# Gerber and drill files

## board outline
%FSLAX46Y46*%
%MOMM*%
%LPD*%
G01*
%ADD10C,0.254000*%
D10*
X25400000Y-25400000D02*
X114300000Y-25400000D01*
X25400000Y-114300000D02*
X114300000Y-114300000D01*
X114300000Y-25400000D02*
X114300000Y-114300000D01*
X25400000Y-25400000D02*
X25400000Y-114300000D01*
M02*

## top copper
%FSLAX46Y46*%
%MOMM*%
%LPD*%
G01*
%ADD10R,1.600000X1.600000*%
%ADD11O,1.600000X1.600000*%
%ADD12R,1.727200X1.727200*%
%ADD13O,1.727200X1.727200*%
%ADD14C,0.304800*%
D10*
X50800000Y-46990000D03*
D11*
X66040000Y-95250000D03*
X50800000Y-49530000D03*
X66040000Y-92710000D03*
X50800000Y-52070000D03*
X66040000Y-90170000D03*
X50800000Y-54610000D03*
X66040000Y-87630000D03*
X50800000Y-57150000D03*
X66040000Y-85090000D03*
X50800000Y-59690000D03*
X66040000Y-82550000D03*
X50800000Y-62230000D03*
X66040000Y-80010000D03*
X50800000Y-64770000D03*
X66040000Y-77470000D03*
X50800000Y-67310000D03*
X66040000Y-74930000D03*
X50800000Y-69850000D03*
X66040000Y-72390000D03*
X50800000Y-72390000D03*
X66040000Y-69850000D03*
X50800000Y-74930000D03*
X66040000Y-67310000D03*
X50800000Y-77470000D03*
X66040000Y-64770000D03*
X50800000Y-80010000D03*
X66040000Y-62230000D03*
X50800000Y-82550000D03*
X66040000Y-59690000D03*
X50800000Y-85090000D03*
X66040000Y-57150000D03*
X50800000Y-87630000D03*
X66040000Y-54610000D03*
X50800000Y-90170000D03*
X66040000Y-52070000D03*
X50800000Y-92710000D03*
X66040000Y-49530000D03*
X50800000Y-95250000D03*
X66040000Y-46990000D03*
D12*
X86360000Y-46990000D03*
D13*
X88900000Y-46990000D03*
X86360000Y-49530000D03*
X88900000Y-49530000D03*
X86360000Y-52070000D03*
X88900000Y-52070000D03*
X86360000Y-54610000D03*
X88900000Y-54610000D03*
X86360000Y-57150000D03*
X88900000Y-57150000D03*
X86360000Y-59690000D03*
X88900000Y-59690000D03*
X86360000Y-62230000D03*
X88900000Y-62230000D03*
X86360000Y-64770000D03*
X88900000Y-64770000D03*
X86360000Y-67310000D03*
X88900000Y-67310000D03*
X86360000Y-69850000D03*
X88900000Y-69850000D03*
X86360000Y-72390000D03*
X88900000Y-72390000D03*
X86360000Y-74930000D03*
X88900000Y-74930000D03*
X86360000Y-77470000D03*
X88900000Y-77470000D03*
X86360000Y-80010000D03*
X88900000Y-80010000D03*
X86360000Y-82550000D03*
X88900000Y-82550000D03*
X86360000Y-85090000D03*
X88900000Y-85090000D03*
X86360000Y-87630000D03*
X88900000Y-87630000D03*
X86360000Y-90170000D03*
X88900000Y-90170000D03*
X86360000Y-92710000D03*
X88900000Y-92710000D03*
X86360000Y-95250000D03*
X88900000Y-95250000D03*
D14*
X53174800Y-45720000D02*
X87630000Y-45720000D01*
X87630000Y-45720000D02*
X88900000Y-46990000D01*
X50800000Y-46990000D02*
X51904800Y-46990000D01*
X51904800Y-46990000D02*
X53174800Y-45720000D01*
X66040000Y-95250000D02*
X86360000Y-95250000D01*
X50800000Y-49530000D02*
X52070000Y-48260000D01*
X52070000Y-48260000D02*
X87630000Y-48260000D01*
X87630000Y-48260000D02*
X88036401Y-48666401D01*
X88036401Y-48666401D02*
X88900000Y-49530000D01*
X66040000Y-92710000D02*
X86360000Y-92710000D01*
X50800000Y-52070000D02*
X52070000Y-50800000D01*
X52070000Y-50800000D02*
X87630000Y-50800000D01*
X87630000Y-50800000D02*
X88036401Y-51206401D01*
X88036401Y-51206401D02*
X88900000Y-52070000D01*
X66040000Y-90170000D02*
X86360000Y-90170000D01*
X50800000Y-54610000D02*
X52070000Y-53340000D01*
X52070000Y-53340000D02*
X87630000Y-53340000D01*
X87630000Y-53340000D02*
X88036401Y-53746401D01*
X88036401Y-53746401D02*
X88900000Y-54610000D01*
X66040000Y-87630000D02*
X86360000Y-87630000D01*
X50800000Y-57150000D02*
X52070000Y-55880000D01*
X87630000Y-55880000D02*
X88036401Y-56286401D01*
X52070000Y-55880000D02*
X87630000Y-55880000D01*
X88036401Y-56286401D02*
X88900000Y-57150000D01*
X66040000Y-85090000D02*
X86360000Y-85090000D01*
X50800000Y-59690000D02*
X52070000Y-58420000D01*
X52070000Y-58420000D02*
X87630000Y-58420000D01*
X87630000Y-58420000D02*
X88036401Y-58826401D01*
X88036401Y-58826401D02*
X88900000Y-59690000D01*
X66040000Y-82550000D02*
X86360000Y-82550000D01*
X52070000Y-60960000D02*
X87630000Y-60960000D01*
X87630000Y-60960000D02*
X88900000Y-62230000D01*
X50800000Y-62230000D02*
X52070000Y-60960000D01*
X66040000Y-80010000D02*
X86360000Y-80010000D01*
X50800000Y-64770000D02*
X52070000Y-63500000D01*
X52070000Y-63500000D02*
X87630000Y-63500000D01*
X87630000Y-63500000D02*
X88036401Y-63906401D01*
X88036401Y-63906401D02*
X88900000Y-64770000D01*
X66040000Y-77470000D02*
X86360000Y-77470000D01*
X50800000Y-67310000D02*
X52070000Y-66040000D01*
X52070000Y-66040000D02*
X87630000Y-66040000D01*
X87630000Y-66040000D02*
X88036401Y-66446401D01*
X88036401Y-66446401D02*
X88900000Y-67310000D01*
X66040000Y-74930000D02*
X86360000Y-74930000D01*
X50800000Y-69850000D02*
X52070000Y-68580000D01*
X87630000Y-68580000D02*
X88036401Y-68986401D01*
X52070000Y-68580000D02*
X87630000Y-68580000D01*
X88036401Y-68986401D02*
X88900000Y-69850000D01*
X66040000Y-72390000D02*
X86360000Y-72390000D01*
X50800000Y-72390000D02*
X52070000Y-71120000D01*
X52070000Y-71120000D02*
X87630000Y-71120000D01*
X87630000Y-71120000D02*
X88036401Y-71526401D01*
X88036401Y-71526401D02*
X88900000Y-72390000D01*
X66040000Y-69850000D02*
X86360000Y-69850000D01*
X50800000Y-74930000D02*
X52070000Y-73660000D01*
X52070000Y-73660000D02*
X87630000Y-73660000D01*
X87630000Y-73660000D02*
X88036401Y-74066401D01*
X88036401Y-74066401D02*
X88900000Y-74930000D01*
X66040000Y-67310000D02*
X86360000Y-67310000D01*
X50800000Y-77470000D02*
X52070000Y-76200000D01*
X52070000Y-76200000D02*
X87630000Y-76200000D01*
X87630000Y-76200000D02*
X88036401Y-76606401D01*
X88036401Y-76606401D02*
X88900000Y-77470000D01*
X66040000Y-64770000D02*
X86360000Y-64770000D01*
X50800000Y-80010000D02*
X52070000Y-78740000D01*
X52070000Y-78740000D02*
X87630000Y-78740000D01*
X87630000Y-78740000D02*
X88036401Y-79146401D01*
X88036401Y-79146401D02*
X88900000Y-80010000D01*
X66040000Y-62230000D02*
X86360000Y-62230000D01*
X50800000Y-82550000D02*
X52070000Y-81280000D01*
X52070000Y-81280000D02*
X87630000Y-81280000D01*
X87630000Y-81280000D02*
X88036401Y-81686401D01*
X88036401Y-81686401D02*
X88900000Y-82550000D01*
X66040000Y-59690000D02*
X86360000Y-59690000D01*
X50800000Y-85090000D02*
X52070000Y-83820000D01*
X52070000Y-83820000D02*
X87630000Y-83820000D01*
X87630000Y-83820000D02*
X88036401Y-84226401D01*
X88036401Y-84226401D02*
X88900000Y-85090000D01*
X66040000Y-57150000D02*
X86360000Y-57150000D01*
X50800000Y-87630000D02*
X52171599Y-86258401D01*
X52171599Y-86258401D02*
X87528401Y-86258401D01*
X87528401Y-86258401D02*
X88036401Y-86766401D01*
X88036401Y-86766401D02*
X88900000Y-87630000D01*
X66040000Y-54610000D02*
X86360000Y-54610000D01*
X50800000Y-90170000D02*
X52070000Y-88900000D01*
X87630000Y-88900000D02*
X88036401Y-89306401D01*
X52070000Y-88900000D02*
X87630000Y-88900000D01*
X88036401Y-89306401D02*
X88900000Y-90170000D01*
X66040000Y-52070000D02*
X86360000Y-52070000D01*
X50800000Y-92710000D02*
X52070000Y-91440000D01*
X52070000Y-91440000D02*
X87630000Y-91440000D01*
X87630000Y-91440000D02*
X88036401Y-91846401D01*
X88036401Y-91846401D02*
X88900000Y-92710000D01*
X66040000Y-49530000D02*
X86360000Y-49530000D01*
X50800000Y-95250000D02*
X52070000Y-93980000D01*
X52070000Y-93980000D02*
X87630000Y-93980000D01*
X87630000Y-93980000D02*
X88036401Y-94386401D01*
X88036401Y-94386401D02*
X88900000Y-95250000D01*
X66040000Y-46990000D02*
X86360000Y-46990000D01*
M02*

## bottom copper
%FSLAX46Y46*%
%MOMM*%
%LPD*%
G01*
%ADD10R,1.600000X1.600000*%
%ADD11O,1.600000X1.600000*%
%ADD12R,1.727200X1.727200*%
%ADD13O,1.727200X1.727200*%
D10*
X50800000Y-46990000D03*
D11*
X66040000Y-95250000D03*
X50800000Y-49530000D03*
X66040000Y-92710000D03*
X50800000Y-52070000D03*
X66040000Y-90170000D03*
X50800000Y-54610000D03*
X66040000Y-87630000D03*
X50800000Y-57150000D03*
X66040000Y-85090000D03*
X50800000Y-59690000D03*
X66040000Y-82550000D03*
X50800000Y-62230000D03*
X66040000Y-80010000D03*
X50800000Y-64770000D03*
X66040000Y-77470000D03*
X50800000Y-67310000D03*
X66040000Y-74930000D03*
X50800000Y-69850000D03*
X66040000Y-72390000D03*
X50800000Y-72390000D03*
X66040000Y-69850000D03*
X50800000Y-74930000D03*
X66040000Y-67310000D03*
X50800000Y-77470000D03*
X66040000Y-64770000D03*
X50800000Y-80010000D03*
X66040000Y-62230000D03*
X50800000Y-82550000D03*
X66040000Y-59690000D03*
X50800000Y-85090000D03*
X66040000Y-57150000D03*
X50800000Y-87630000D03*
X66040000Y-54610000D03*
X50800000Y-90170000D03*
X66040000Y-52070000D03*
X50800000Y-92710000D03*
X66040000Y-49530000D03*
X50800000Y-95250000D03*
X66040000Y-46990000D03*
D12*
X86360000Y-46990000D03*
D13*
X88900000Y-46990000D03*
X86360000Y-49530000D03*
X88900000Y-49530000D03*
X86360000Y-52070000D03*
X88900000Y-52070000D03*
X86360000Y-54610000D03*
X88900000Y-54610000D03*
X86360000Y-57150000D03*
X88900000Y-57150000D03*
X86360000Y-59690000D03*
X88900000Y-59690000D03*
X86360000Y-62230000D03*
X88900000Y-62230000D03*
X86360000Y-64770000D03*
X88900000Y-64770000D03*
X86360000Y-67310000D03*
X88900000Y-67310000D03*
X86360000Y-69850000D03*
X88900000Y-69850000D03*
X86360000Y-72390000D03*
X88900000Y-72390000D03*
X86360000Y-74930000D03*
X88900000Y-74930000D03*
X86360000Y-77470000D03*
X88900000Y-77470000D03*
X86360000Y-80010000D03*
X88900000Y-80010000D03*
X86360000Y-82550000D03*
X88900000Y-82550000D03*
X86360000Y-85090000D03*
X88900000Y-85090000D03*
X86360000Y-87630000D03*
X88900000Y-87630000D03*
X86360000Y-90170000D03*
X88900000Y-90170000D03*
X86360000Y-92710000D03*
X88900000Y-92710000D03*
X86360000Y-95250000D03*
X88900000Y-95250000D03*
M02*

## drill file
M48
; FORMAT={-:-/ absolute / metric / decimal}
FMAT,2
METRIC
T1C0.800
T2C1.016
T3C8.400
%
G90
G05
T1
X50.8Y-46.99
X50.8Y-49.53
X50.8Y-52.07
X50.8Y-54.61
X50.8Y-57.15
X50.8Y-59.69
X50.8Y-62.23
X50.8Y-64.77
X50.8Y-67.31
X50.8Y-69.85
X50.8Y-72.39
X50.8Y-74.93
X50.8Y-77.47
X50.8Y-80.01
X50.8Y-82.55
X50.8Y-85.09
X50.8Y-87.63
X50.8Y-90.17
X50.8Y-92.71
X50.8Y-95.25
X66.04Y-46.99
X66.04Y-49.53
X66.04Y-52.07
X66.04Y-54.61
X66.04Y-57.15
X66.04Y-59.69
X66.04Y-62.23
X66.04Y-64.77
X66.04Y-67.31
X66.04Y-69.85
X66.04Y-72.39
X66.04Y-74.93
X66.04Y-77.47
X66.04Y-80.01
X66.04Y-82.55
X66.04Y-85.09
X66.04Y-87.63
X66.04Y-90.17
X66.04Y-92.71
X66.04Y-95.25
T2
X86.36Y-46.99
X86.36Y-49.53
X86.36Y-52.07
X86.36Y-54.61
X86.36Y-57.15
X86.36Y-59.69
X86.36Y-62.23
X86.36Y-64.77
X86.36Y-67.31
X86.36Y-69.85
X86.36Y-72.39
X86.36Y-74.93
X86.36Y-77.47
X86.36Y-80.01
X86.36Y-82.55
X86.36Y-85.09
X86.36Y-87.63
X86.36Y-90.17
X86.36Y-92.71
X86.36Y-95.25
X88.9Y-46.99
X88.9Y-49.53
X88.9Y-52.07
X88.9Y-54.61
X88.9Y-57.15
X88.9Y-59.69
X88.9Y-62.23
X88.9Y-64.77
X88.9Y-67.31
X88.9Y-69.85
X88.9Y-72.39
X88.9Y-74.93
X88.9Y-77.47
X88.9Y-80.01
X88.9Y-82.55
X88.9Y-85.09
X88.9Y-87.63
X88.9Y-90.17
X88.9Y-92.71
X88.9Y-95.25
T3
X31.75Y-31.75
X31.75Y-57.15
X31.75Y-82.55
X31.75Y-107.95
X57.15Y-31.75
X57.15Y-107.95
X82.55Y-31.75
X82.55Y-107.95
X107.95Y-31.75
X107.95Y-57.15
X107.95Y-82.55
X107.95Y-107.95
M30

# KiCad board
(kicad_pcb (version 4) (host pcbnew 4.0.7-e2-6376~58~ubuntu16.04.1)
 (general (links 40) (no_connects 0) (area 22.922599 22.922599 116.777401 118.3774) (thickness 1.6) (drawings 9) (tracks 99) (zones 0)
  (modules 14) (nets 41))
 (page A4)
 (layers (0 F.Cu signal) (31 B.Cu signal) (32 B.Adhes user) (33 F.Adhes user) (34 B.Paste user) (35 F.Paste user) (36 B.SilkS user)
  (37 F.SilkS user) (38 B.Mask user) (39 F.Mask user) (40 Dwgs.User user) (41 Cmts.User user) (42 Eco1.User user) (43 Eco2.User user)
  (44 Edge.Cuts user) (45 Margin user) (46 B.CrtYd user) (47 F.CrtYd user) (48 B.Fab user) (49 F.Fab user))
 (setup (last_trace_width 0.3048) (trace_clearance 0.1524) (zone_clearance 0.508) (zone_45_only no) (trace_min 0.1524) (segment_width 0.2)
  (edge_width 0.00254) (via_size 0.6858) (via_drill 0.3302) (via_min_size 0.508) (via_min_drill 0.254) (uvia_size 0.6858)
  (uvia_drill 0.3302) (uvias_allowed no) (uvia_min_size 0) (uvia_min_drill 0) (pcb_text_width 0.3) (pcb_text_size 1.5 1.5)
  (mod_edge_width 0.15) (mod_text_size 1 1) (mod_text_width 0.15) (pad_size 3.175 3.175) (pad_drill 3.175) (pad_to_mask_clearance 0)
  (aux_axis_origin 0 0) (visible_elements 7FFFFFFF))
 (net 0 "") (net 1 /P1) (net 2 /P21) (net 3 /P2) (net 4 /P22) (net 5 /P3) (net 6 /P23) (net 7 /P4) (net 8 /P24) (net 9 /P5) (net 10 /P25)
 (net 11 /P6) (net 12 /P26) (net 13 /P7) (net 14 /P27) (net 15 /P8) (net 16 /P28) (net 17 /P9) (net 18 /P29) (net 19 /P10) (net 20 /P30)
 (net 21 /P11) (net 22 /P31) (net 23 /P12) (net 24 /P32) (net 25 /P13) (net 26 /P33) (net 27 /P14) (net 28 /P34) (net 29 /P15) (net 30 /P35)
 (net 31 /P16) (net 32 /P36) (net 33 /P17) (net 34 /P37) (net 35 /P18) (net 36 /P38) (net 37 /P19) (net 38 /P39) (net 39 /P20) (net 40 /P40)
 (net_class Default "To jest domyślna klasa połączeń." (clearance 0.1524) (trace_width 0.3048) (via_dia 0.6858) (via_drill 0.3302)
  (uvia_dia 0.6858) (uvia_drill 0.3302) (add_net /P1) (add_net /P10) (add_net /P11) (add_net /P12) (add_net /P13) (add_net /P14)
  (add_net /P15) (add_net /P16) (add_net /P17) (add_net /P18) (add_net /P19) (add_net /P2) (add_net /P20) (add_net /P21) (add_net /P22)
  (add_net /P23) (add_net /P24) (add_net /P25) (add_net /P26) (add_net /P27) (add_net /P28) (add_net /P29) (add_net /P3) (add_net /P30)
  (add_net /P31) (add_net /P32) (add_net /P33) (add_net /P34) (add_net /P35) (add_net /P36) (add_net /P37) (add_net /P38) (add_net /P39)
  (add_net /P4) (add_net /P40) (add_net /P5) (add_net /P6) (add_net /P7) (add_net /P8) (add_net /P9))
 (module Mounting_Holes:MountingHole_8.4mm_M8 (layer F.Cu) (at 82.55 107.95)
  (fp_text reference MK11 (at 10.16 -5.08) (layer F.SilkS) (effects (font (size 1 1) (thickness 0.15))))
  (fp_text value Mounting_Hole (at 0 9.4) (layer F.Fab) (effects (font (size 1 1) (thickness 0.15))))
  (pad 1 np_thru_hole circle (at 0 0) (size 8.4 8.4) (drill 8.4) (layers *.Cu *.Mask)))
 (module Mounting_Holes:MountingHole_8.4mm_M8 (layer F.Cu) (at 57.15 107.95)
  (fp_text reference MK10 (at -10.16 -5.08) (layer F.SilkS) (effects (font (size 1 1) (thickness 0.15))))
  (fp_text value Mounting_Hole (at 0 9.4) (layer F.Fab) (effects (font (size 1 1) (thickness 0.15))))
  (pad 1 np_thru_hole circle (at 0 0) (size 8.4 8.4) (drill 8.4) (layers *.Cu *.Mask)))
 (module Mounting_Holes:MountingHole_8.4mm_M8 (layer F.Cu) (at 107.95 82.55)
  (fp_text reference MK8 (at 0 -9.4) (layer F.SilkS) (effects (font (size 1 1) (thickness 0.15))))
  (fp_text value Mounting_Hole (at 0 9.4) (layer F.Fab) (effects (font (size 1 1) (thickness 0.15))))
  (pad 1 np_thru_hole circle (at 0 0) (size 8.4 8.4) (drill 8.4) (layers *.Cu *.Mask)))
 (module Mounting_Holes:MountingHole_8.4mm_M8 (layer F.Cu) (at 107.95 57.15)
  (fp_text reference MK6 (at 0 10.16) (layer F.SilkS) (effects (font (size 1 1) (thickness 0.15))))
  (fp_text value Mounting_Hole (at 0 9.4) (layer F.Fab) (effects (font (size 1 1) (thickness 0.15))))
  (pad 1 np_thru_hole circle (at 0 0) (size 8.4 8.4) (drill 8.4) (layers *.Cu *.Mask)))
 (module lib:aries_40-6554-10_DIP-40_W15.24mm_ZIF (layer F.Cu) (at 50.8 46.99)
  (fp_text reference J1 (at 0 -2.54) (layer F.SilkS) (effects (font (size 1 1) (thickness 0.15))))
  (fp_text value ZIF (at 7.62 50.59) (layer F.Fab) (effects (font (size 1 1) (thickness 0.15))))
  (pad 1 thru_hole rect (at 0 0) (size 1.6 1.6) (drill 0.8) (layers *.Cu *.Mask) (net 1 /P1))
  (pad 21 thru_hole oval (at 15.24 48.26) (size 1.6 1.6) (drill 0.8) (layers *.Cu *.Mask) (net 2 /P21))
  (pad 2 thru_hole oval (at 0 2.54) (size 1.6 1.6) (drill 0.8) (layers *.Cu *.Mask) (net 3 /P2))
  (pad 22 thru_hole oval (at 15.24 45.72) (size 1.6 1.6) (drill 0.8) (layers *.Cu *.Mask) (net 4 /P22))
  (pad 3 thru_hole oval (at 0 5.08) (size 1.6 1.6) (drill 0.8) (layers *.Cu *.Mask) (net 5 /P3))
  (pad 23 thru_hole oval (at 15.24 43.18) (size 1.6 1.6) (drill 0.8) (layers *.Cu *.Mask) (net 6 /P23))
  (pad 4 thru_hole oval (at 0 7.62) (size 1.6 1.6) (drill 0.8) (layers *.Cu *.Mask) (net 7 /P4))
  (pad 24 thru_hole oval (at 15.24 40.64) (size 1.6 1.6) (drill 0.8) (layers *.Cu *.Mask) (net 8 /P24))
  (pad 5 thru_hole oval (at 0 10.16) (size 1.6 1.6) (drill 0.8) (layers *.Cu *.Mask) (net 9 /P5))
  (pad 25 thru_hole oval (at 15.24 38.1) (size 1.6 1.6) (drill 0.8) (layers *.Cu *.Mask) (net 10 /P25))
  (pad 6 thru_hole oval (at 0 12.7) (size 1.6 1.6) (drill 0.8) (layers *.Cu *.Mask) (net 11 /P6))
  (pad 26 thru_hole oval (at 15.24 35.56) (size 1.6 1.6) (drill 0.8) (layers *.Cu *.Mask) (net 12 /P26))
  (pad 7 thru_hole oval (at 0 15.24) (size 1.6 1.6) (drill 0.8) (layers *.Cu *.Mask) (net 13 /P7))
  (pad 27 thru_hole oval (at 15.24 33.02) (size 1.6 1.6) (drill 0.8) (layers *.Cu *.Mask) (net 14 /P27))
  (pad 8 thru_hole oval (at 0 17.78) (size 1.6 1.6) (drill 0.8) (layers *.Cu *.Mask) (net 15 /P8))
  (pad 28 thru_hole oval (at 15.24 30.48) (size 1.6 1.6) (drill 0.8) (layers *.Cu *.Mask) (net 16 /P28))
  (pad 9 thru_hole oval (at 0 20.32) (size 1.6 1.6) (drill 0.8) (layers *.Cu *.Mask) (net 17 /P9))
  (pad 29 thru_hole oval (at 15.24 27.94) (size 1.6 1.6) (drill 0.8) (layers *.Cu *.Mask) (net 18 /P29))
  (pad 10 thru_hole oval (at 0 22.86) (size 1.6 1.6) (drill 0.8) (layers *.Cu *.Mask) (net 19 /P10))
  (pad 30 thru_hole oval (at 15.24 25.4) (size 1.6 1.6) (drill 0.8) (layers *.Cu *.Mask) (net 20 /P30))
  (pad 11 thru_hole oval (at 0 25.4) (size 1.6 1.6) (drill 0.8) (layers *.Cu *.Mask) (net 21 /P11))
  (pad 31 thru_hole oval (at 15.24 22.86) (size 1.6 1.6) (drill 0.8) (layers *.Cu *.Mask) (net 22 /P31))
  (pad 12 thru_hole oval (at 0 27.94) (size 1.6 1.6) (drill 0.8) (layers *.Cu *.Mask) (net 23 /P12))
  (pad 32 thru_hole oval (at 15.24 20.32) (size 1.6 1.6) (drill 0.8) (layers *.Cu *.Mask) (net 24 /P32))
  (pad 13 thru_hole oval (at 0 30.48) (size 1.6 1.6) (drill 0.8) (layers *.Cu *.Mask) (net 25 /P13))
  (pad 33 thru_hole oval (at 15.24 17.78) (size 1.6 1.6) (drill 0.8) (layers *.Cu *.Mask) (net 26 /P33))
  (pad 14 thru_hole oval (at 0 33.02) (size 1.6 1.6) (drill 0.8) (layers *.Cu *.Mask) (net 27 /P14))
  (pad 34 thru_hole oval (at 15.24 15.24) (size 1.6 1.6) (drill 0.8) (layers *.Cu *.Mask) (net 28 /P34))
  (pad 15 thru_hole oval (at 0 35.56) (size 1.6 1.6) (drill 0.8) (layers *.Cu *.Mask) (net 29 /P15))
  (pad 35 thru_hole oval (at 15.24 12.7) (size 1.6 1.6) (drill 0.8) (layers *.Cu *.Mask) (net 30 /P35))
  (pad 16 thru_hole oval (at 0 38.1) (size 1.6 1.6) (drill 0.8) (layers *.Cu *.Mask) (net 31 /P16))
  (pad 36 thru_hole oval (at 15.24 10.16) (size 1.6 1.6) (drill 0.8) (layers *.Cu *.Mask) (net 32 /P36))
  (pad 17 thru_hole oval (at 0 40.64) (size 1.6 1.6) (drill 0.8) (layers *.Cu *.Mask) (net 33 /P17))
  (pad 37 thru_hole oval (at 15.24 7.62) (size 1.6 1.6) (drill 0.8) (layers *.Cu *.Mask) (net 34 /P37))
  (pad 18 thru_hole oval (at 0 43.18) (size 1.6 1.6) (drill 0.8) (layers *.Cu *.Mask) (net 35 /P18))
  (pad 38 thru_hole oval (at 15.24 5.08) (size 1.6 1.6) (drill 0.8) (layers *.Cu *.Mask) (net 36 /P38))
  (pad 19 thru_hole oval (at 0 45.72) (size 1.6 1.6) (drill 0.8) (layers *.Cu *.Mask) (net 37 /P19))
  (pad 39 thru_hole oval (at 15.24 2.54) (size 1.6 1.6) (drill 0.8) (layers *.Cu *.Mask) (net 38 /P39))
  (pad 20 thru_hole oval (at 0 48.26) (size 1.6 1.6) (drill 0.8) (layers *.Cu *.Mask) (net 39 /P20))
  (pad 40 thru_hole oval (at 15.24 0) (size 1.6 1.6) (drill 0.8) (layers *.Cu *.Mask) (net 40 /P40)))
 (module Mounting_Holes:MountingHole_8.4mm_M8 (layer F.Cu) (at 31.75 31.75)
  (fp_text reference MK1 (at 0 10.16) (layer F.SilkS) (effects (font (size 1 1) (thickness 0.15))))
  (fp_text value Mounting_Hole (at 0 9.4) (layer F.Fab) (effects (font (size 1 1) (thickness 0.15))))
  (pad 1 np_thru_hole circle (at 0 0) (size 8.4 8.4) (drill 8.4) (layers *.Cu *.Mask)))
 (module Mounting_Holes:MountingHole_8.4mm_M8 (layer F.Cu) (at 107.95 31.75)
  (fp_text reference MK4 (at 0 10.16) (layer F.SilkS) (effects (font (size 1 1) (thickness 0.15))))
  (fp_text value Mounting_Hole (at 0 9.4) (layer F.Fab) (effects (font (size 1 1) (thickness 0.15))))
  (pad 1 np_thru_hole circle (at 0 0) (size 8.4 8.4) (drill 8.4) (layers *.Cu *.Mask)))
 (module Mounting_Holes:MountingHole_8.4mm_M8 (layer F.Cu) (at 31.75 107.95)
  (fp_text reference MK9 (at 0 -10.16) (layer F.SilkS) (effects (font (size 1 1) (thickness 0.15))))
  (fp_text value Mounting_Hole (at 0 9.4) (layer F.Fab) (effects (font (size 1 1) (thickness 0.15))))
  (pad 1 np_thru_hole circle (at 0 0) (size 8.4 8.4) (drill 8.4) (layers *.Cu *.Mask)))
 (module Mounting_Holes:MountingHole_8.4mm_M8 (layer F.Cu) (at 107.95 107.95)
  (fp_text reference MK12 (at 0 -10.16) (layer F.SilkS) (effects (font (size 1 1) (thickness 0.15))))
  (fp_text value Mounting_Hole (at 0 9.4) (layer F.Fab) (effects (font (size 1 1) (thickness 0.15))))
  (pad 1 np_thru_hole circle (at 0 0) (size 8.4 8.4) (drill 8.4) (layers *.Cu *.Mask)))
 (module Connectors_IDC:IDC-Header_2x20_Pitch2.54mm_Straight (layer F.Cu) (at 86.36 46.99)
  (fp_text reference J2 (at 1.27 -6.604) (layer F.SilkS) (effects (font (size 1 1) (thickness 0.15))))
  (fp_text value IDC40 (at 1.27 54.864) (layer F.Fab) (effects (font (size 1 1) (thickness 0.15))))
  (pad 1 thru_hole rect (at 0 0) (size 1.7272 1.7272) (drill 1.016) (layers *.Cu *.Mask) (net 40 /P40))
  (pad 2 thru_hole oval (at 2.54 0) (size 1.7272 1.7272) (drill 1.016) (layers *.Cu *.Mask) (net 1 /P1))
  (pad 3 thru_hole oval (at 0 2.54) (size 1.7272 1.7272) (drill 1.016) (layers *.Cu *.Mask) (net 38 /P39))
  (pad 4 thru_hole oval (at 2.54 2.54) (size 1.7272 1.7272) (drill 1.016) (layers *.Cu *.Mask) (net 3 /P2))
  (pad 5 thru_hole oval (at 0 5.08) (size 1.7272 1.7272) (drill 1.016) (layers *.Cu *.Mask) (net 36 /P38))
  (pad 6 thru_hole oval (at 2.54 5.08) (size 1.7272 1.7272) (drill 1.016) (layers *.Cu *.Mask) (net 5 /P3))
  (pad 7 thru_hole oval (at 0 7.62) (size 1.7272 1.7272) (drill 1.016) (layers *.Cu *.Mask) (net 34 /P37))
  (pad 8 thru_hole oval (at 2.54 7.62) (size 1.7272 1.7272) (drill 1.016) (layers *.Cu *.Mask) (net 7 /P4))
  (pad 9 thru_hole oval (at 0 10.16) (size 1.7272 1.7272) (drill 1.016) (layers *.Cu *.Mask) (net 32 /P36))
  (pad 10 thru_hole oval (at 2.54 10.16) (size 1.7272 1.7272) (drill 1.016) (layers *.Cu *.Mask) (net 9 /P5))
  (pad 11 thru_hole oval (at 0 12.7) (size 1.7272 1.7272) (drill 1.016) (layers *.Cu *.Mask) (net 30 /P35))
  (pad 12 thru_hole oval (at 2.54 12.7) (size 1.7272 1.7272) (drill 1.016) (layers *.Cu *.Mask) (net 11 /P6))
  (pad 13 thru_hole oval (at 0 15.24) (size 1.7272 1.7272) (drill 1.016) (layers *.Cu *.Mask) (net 28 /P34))
  (pad 14 thru_hole oval (at 2.54 15.24) (size 1.7272 1.7272) (drill 1.016) (layers *.Cu *.Mask) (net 13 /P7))
  (pad 15 thru_hole oval (at 0 17.78) (size 1.7272 1.7272) (drill 1.016) (layers *.Cu *.Mask) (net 26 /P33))
  (pad 16 thru_hole oval (at 2.54 17.78) (size 1.7272 1.7272) (drill 1.016) (layers *.Cu *.Mask) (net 15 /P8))
  (pad 17 thru_hole oval (at 0 20.32) (size 1.7272 1.7272) (drill 1.016) (layers *.Cu *.Mask) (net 24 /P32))
  (pad 18 thru_hole oval (at 2.54 20.32) (size 1.7272 1.7272) (drill 1.016) (layers *.Cu *.Mask) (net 17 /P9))
  (pad 19 thru_hole oval (at 0 22.86) (size 1.7272 1.7272) (drill 1.016) (layers *.Cu *.Mask) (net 22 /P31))
  (pad 20 thru_hole oval (at 2.54 22.86) (size 1.7272 1.7272) (drill 1.016) (layers *.Cu *.Mask) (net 19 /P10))
  (pad 21 thru_hole oval (at 0 25.4) (size 1.7272 1.7272) (drill 1.016) (layers *.Cu *.Mask) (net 20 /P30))
  (pad 22 thru_hole oval (at 2.54 25.4) (size 1.7272 1.7272) (drill 1.016) (layers *.Cu *.Mask) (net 21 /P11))
  (pad 23 thru_hole oval (at 0 27.94) (size 1.7272 1.7272) (drill 1.016) (layers *.Cu *.Mask) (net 18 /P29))
  (pad 24 thru_hole oval (at 2.54 27.94) (size 1.7272 1.7272) (drill 1.016) (layers *.Cu *.Mask) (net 23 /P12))
  (pad 25 thru_hole oval (at 0 30.48) (size 1.7272 1.7272) (drill 1.016) (layers *.Cu *.Mask) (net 16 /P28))
  (pad 26 thru_hole oval (at 2.54 30.48) (size 1.7272 1.7272) (drill 1.016) (layers *.Cu *.Mask) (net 25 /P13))
  (pad 27 thru_hole oval (at 0 33.02) (size 1.7272 1.7272) (drill 1.016) (layers *.Cu *.Mask) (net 14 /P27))
  (pad 28 thru_hole oval (at 2.54 33.02) (size 1.7272 1.7272) (drill 1.016) (layers *.Cu *.Mask) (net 27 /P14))
  (pad 29 thru_hole oval (at 0 35.56) (size 1.7272 1.7272) (drill 1.016) (layers *.Cu *.Mask) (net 12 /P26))
  (pad 30 thru_hole oval (at 2.54 35.56) (size 1.7272 1.7272) (drill 1.016) (layers *.Cu *.Mask) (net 29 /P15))
  (pad 31 thru_hole oval (at 0 38.1) (size 1.7272 1.7272) (drill 1.016) (layers *.Cu *.Mask) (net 10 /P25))
  (pad 32 thru_hole oval (at 2.54 38.1) (size 1.7272 1.7272) (drill 1.016) (layers *.Cu *.Mask) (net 31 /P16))
  (pad 33 thru_hole oval (at 0 40.64) (size 1.7272 1.7272) (drill 1.016) (layers *.Cu *.Mask) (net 8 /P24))
  (pad 34 thru_hole oval (at 2.54 40.64) (size 1.7272 1.7272) (drill 1.016) (layers *.Cu *.Mask) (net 33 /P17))
  (pad 35 thru_hole oval (at 0 43.18) (size 1.7272 1.7272) (drill 1.016) (layers *.Cu *.Mask) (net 6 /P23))
  (pad 36 thru_hole oval (at 2.54 43.18) (size 1.7272 1.7272) (drill 1.016) (layers *.Cu *.Mask) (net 35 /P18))
  (pad 37 thru_hole oval (at 0 45.72) (size 1.7272 1.7272) (drill 1.016) (layers *.Cu *.Mask) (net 4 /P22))
  (pad 38 thru_hole oval (at 2.54 45.72) (size 1.7272 1.7272) (drill 1.016) (layers *.Cu *.Mask) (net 37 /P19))
  (pad 39 thru_hole oval (at 0 48.26) (size 1.7272 1.7272) (drill 1.016) (layers *.Cu *.Mask) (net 2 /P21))
  (pad 40 thru_hole oval (at 2.54 48.26) (size 1.7272 1.7272) (drill 1.016) (layers *.Cu *.Mask) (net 39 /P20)))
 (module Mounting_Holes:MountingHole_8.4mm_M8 (layer F.Cu) (at 82.55 31.75)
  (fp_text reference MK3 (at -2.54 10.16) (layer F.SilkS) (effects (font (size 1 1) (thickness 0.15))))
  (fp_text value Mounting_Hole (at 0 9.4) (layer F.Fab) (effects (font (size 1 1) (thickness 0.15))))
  (pad 1 np_thru_hole circle (at 0 0) (size 8.4 8.4) (drill 8.4) (layers *.Cu *.Mask)))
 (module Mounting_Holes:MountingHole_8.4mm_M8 (layer F.Cu) (at 57.15 31.75)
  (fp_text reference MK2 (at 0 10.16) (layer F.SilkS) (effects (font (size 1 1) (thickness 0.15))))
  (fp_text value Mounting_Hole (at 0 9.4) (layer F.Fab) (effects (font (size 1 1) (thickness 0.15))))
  (pad 1 np_thru_hole circle (at 0 0) (size 8.4 8.4) (drill 8.4) (layers *.Cu *.Mask)))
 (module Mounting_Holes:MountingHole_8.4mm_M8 (layer F.Cu) (at 31.75 57.15)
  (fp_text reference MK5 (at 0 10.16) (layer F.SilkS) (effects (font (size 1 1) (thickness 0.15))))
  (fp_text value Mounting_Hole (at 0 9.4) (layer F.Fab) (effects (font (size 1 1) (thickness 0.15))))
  (pad 1 np_thru_hole circle (at 0 0) (size 8.4 8.4) (drill 8.4) (layers *.Cu *.Mask)))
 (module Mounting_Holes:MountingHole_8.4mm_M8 (layer F.Cu) (at 31.75 82.55)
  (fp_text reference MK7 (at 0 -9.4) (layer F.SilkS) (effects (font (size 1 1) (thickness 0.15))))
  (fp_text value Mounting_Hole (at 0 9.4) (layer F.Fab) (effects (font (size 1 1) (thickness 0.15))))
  (pad 1 np_thru_hole circle (at 0 0) (size 8.4 8.4) (drill 8.4) (layers *.Cu *.Mask)))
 (gr_line (start 25.4 25.4) (end 114.3 25.4) (layer Edge.Cuts) (width 0.254))
 (gr_line (start 25.4 114.3) (end 114.3 114.3) (layer Edge.Cuts) (width 0.254))
 (gr_line (start 114.3 25.4) (end 114.3 114.3) (layer Edge.Cuts) (width 0.254))
 (gr_line (start 25.4 25.4) (end 25.4 114.3) (layer Edge.Cuts) (width 0.254))
 (segment (start 53.1748 45.72) (end 87.63 45.72) (width 0.3048) (layer F.Cu) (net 1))
 (segment (start 87.63 45.72) (end 88.9 46.99) (width 0.3048) (layer F.Cu) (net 1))
 (segment (start 50.8 46.99) (end 51.9048 46.99) (width 0.3048) (layer F.Cu) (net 1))
 (segment (start 51.9048 46.99) (end 53.1748 45.72) (width 0.3048) (layer F.Cu) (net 1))
 (segment (start 66.04 95.25) (end 86.36 95.25) (width 0.3048) (layer F.Cu) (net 2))
 (segment (start 50.8 49.53) (end 52.07 48.26) (width 0.3048) (layer F.Cu) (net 3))
 (segment (start 52.07 48.26) (end 87.63 48.26) (width 0.3048) (layer F.Cu) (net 3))
 (segment (start 87.63 48.26) (end 88.036401 48.666401) (width 0.3048) (layer F.Cu) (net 3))
 (segment (start 88.036401 48.666401) (end 88.9 49.53) (width 0.3048) (layer F.Cu) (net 3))
 (segment (start 66.04 92.71) (end 86.36 92.71) (width 0.3048) (layer F.Cu) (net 4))
 (segment (start 50.8 52.07) (end 52.07 50.8) (width 0.3048) (layer F.Cu) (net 5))
 (segment (start 52.07 50.8) (end 87.63 50.8) (width 0.3048) (layer F.Cu) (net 5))
 (segment (start 87.63 50.8) (end 88.036401 51.206401) (width 0.3048) (layer F.Cu) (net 5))
 (segment (start 88.036401 51.206401) (end 88.9 52.07) (width 0.3048) (layer F.Cu) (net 5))
 (segment (start 66.04 90.17) (end 86.36 90.17) (width 0.3048) (layer F.Cu) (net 6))
 (segment (start 50.8 54.61) (end 52.07 53.34) (width 0.3048) (layer F.Cu) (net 7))
 (segment (start 52.07 53.34) (end 87.63 53.34) (width 0.3048) (layer F.Cu) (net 7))
 (segment (start 87.63 53.34) (end 88.036401 53.746401) (width 0.3048) (layer F.Cu) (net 7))
 (segment (start 88.036401 53.746401) (end 88.9 54.61) (width 0.3048) (layer F.Cu) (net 7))
 (segment (start 66.04 87.63) (end 86.36 87.63) (width 0.3048) (layer F.Cu) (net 8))
 (segment (start 50.8 57.15) (end 52.07 55.88) (width 0.3048) (layer F.Cu) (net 9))
 (segment (start 87.63 55.88) (end 88.036401 56.286401) (width 0.3048) (layer F.Cu) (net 9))
 (segment (start 52.07 55.88) (end 87.63 55.88) (width 0.3048) (layer F.Cu) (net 9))
 (segment (start 88.036401 56.286401) (end 88.9 57.15) (width 0.3048) (layer F.Cu) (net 9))
 (segment (start 66.04 85.09) (end 86.36 85.09) (width 0.3048) (layer F.Cu) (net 10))
 (segment (start 50.8 59.69) (end 52.07 58.42) (width 0.3048) (layer F.Cu) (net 11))
 (segment (start 52.07 58.42) (end 87.63 58.42) (width 0.3048) (layer F.Cu) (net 11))
 (segment (start 87.63 58.42) (end 88.036401 58.826401) (width 0.3048) (layer F.Cu) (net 11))
 (segment (start 88.036401 58.826401) (end 88.9 59.69) (width 0.3048) (layer F.Cu) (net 11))
 (segment (start 66.04 82.55) (end 86.36 82.55) (width 0.3048) (layer F.Cu) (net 12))
 (segment (start 52.07 60.96) (end 87.63 60.96) (width 0.3048) (layer F.Cu) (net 13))
 (segment (start 87.63 60.96) (end 88.9 62.23) (width 0.3048) (layer F.Cu) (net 13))
 (segment (start 50.8 62.23) (end 52.07 60.96) (width 0.3048) (layer F.Cu) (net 13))
 (segment (start 66.04 80.01) (end 86.36 80.01) (width 0.3048) (layer F.Cu) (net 14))
 (segment (start 50.8 64.77) (end 52.07 63.5) (width 0.3048) (layer F.Cu) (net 15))
 (segment (start 52.07 63.5) (end 87.63 63.5) (width 0.3048) (layer F.Cu) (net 15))
 (segment (start 87.63 63.5) (end 88.036401 63.906401) (width 0.3048) (layer F.Cu) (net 15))
 (segment (start 88.036401 63.906401) (end 88.9 64.77) (width 0.3048) (layer F.Cu) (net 15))
 (segment (start 66.04 77.47) (end 86.36 77.47) (width 0.3048) (layer F.Cu) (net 16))
 (segment (start 50.8 67.31) (end 52.07 66.04) (width 0.3048) (layer F.Cu) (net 17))
 (segment (start 52.07 66.04) (end 87.63 66.04) (width 0.3048) (layer F.Cu) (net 17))
 (segment (start 87.63 66.04) (end 88.036401 66.446401) (width 0.3048) (layer F.Cu) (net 17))
 (segment (start 88.036401 66.446401) (end 88.9 67.31) (width 0.3048) (layer F.Cu) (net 17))
 (segment (start 66.04 74.93) (end 86.36 74.93) (width 0.3048) (layer F.Cu) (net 18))
 (segment (start 50.8 69.85) (end 52.07 68.58) (width 0.3048) (layer F.Cu) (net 19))
 (segment (start 87.63 68.58) (end 88.036401 68.986401) (width 0.3048) (layer F.Cu) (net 19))
 (segment (start 52.07 68.58) (end 87.63 68.58) (width 0.3048) (layer F.Cu) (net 19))
 (segment (start 88.036401 68.986401) (end 88.9 69.85) (width 0.3048) (layer F.Cu) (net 19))
 (segment (start 66.04 72.39) (end 86.36 72.39) (width 0.3048) (layer F.Cu) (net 20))
 (segment (start 50.8 72.39) (end 52.07 71.12) (width 0.3048) (layer F.Cu) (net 21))
 (segment (start 52.07 71.12) (end 87.63 71.12) (width 0.3048) (layer F.Cu) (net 21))
 (segment (start 87.63 71.12) (end 88.036401 71.526401) (width 0.3048) (layer F.Cu) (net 21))
 (segment (start 88.036401 71.526401) (end 88.9 72.39) (width 0.3048) (layer F.Cu) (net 21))
 (segment (start 66.04 69.85) (end 86.36 69.85) (width 0.3048) (layer F.Cu) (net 22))
 (segment (start 50.8 74.93) (end 52.07 73.66) (width 0.3048) (layer F.Cu) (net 23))
 (segment (start 52.07 73.66) (end 87.63 73.66) (width 0.3048) (layer F.Cu) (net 23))
 (segment (start 87.63 73.66) (end 88.036401 74.066401) (width 0.3048) (layer F.Cu) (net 23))
 (segment (start 88.036401 74.066401) (end 88.9 74.93) (width 0.3048) (layer F.Cu) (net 23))
 (segment (start 66.04 67.31) (end 86.36 67.31) (width 0.3048) (layer F.Cu) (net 24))
 (segment (start 50.8 77.47) (end 52.07 76.2) (width 0.3048) (layer F.Cu) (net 25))
 (segment (start 52.07 76.2) (end 87.63 76.2) (width 0.3048) (layer F.Cu) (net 25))
 (segment (start 87.63 76.2) (end 88.036401 76.606401) (width 0.3048) (layer F.Cu) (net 25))
 (segment (start 88.036401 76.606401) (end 88.9 77.47) (width 0.3048) (layer F.Cu) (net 25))
 (segment (start 66.04 64.77) (end 86.36 64.77) (width 0.3048) (layer F.Cu) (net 26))
 (segment (start 50.8 80.01) (end 52.07 78.74) (width 0.3048) (layer F.Cu) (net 27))
 (segment (start 52.07 78.74) (end 87.63 78.74) (width 0.3048) (layer F.Cu) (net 27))
 (segment (start 87.63 78.74) (end 88.036401 79.146401) (width 0.3048) (layer F.Cu) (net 27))
 (segment (start 88.036401 79.146401) (end 88.9 80.01) (width 0.3048) (layer F.Cu) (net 27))
 (segment (start 66.04 62.23) (end 86.36 62.23) (width 0.3048) (layer F.Cu) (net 28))
 (segment (start 50.8 82.55) (end 52.07 81.28) (width 0.3048) (layer F.Cu) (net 29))
 (segment (start 52.07 81.28) (end 87.63 81.28) (width 0.3048) (layer F.Cu) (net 29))
 (segment (start 87.63 81.28) (end 88.036401 81.686401) (width 0.3048) (layer F.Cu) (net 29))
 (segment (start 88.036401 81.686401) (end 88.9 82.55) (width 0.3048) (layer F.Cu) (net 29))
 (segment (start 66.04 59.69) (end 86.36 59.69) (width 0.3048) (layer F.Cu) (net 30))
 (segment (start 50.8 85.09) (end 52.07 83.82) (width 0.3048) (layer F.Cu) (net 31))
 (segment (start 52.07 83.82) (end 87.63 83.82) (width 0.3048) (layer F.Cu) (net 31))
 (segment (start 87.63 83.82) (end 88.036401 84.226401) (width 0.3048) (layer F.Cu) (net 31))
 (segment (start 88.036401 84.226401) (end 88.9 85.09) (width 0.3048) (layer F.Cu) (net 31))
 (segment (start 66.04 57.15) (end 86.36 57.15) (width 0.3048) (layer F.Cu) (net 32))
 (segment (start 50.8 87.63) (end 52.171599 86.258401) (width 0.3048) (layer F.Cu) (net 33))
 (segment (start 52.171599 86.258401) (end 87.528401 86.258401) (width 0.3048) (layer F.Cu) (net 33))
 (segment (start 87.528401 86.258401) (end 88.036401 86.766401) (width 0.3048) (layer F.Cu) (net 33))
 (segment (start 88.036401 86.766401) (end 88.9 87.63) (width 0.3048) (layer F.Cu) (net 33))
 (segment (start 66.04 54.61) (end 86.36 54.61) (width 0.3048) (layer F.Cu) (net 34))
 (segment (start 50.8 90.17) (end 52.07 88.9) (width 0.3048) (layer F.Cu) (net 35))
 (segment (start 87.63 88.9) (end 88.036401 89.306401) (width 0.3048) (layer F.Cu) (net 35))
 (segment (start 52.07 88.9) (end 87.63 88.9) (width 0.3048) (layer F.Cu) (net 35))
 (segment (start 88.036401 89.306401) (end 88.9 90.17) (width 0.3048) (layer F.Cu) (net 35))
 (segment (start 66.04 52.07) (end 86.36 52.07) (width 0.3048) (layer F.Cu) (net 36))
 (segment (start 50.8 92.71) (end 52.07 91.44) (width 0.3048) (layer F.Cu) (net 37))
 (segment (start 52.07 91.44) (end 87.63 91.44) (width 0.3048) (layer F.Cu) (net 37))
 (segment (start 87.63 91.44) (end 88.036401 91.846401) (width 0.3048) (layer F.Cu) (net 37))
 (segment (start 88.036401 91.846401) (end 88.9 92.71) (width 0.3048) (layer F.Cu) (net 37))
 (segment (start 66.04 49.53) (end 86.36 49.53) (width 0.3048) (layer F.Cu) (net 38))
 (segment (start 50.8 95.25) (end 52.07 93.98) (width 0.3048) (layer F.Cu) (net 39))
 (segment (start 52.07 93.98) (end 87.63 93.98) (width 0.3048) (layer F.Cu) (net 39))
 (segment (start 87.63 93.98) (end 88.036401 94.386401) (width 0.3048) (layer F.Cu) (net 39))
 (segment (start 88.036401 94.386401) (end 88.9 95.25) (width 0.3048) (layer F.Cu) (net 39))
 (segment (start 66.04 46.99) (end 86.36 46.99) (width 0.3048) (layer F.Cu) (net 40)))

